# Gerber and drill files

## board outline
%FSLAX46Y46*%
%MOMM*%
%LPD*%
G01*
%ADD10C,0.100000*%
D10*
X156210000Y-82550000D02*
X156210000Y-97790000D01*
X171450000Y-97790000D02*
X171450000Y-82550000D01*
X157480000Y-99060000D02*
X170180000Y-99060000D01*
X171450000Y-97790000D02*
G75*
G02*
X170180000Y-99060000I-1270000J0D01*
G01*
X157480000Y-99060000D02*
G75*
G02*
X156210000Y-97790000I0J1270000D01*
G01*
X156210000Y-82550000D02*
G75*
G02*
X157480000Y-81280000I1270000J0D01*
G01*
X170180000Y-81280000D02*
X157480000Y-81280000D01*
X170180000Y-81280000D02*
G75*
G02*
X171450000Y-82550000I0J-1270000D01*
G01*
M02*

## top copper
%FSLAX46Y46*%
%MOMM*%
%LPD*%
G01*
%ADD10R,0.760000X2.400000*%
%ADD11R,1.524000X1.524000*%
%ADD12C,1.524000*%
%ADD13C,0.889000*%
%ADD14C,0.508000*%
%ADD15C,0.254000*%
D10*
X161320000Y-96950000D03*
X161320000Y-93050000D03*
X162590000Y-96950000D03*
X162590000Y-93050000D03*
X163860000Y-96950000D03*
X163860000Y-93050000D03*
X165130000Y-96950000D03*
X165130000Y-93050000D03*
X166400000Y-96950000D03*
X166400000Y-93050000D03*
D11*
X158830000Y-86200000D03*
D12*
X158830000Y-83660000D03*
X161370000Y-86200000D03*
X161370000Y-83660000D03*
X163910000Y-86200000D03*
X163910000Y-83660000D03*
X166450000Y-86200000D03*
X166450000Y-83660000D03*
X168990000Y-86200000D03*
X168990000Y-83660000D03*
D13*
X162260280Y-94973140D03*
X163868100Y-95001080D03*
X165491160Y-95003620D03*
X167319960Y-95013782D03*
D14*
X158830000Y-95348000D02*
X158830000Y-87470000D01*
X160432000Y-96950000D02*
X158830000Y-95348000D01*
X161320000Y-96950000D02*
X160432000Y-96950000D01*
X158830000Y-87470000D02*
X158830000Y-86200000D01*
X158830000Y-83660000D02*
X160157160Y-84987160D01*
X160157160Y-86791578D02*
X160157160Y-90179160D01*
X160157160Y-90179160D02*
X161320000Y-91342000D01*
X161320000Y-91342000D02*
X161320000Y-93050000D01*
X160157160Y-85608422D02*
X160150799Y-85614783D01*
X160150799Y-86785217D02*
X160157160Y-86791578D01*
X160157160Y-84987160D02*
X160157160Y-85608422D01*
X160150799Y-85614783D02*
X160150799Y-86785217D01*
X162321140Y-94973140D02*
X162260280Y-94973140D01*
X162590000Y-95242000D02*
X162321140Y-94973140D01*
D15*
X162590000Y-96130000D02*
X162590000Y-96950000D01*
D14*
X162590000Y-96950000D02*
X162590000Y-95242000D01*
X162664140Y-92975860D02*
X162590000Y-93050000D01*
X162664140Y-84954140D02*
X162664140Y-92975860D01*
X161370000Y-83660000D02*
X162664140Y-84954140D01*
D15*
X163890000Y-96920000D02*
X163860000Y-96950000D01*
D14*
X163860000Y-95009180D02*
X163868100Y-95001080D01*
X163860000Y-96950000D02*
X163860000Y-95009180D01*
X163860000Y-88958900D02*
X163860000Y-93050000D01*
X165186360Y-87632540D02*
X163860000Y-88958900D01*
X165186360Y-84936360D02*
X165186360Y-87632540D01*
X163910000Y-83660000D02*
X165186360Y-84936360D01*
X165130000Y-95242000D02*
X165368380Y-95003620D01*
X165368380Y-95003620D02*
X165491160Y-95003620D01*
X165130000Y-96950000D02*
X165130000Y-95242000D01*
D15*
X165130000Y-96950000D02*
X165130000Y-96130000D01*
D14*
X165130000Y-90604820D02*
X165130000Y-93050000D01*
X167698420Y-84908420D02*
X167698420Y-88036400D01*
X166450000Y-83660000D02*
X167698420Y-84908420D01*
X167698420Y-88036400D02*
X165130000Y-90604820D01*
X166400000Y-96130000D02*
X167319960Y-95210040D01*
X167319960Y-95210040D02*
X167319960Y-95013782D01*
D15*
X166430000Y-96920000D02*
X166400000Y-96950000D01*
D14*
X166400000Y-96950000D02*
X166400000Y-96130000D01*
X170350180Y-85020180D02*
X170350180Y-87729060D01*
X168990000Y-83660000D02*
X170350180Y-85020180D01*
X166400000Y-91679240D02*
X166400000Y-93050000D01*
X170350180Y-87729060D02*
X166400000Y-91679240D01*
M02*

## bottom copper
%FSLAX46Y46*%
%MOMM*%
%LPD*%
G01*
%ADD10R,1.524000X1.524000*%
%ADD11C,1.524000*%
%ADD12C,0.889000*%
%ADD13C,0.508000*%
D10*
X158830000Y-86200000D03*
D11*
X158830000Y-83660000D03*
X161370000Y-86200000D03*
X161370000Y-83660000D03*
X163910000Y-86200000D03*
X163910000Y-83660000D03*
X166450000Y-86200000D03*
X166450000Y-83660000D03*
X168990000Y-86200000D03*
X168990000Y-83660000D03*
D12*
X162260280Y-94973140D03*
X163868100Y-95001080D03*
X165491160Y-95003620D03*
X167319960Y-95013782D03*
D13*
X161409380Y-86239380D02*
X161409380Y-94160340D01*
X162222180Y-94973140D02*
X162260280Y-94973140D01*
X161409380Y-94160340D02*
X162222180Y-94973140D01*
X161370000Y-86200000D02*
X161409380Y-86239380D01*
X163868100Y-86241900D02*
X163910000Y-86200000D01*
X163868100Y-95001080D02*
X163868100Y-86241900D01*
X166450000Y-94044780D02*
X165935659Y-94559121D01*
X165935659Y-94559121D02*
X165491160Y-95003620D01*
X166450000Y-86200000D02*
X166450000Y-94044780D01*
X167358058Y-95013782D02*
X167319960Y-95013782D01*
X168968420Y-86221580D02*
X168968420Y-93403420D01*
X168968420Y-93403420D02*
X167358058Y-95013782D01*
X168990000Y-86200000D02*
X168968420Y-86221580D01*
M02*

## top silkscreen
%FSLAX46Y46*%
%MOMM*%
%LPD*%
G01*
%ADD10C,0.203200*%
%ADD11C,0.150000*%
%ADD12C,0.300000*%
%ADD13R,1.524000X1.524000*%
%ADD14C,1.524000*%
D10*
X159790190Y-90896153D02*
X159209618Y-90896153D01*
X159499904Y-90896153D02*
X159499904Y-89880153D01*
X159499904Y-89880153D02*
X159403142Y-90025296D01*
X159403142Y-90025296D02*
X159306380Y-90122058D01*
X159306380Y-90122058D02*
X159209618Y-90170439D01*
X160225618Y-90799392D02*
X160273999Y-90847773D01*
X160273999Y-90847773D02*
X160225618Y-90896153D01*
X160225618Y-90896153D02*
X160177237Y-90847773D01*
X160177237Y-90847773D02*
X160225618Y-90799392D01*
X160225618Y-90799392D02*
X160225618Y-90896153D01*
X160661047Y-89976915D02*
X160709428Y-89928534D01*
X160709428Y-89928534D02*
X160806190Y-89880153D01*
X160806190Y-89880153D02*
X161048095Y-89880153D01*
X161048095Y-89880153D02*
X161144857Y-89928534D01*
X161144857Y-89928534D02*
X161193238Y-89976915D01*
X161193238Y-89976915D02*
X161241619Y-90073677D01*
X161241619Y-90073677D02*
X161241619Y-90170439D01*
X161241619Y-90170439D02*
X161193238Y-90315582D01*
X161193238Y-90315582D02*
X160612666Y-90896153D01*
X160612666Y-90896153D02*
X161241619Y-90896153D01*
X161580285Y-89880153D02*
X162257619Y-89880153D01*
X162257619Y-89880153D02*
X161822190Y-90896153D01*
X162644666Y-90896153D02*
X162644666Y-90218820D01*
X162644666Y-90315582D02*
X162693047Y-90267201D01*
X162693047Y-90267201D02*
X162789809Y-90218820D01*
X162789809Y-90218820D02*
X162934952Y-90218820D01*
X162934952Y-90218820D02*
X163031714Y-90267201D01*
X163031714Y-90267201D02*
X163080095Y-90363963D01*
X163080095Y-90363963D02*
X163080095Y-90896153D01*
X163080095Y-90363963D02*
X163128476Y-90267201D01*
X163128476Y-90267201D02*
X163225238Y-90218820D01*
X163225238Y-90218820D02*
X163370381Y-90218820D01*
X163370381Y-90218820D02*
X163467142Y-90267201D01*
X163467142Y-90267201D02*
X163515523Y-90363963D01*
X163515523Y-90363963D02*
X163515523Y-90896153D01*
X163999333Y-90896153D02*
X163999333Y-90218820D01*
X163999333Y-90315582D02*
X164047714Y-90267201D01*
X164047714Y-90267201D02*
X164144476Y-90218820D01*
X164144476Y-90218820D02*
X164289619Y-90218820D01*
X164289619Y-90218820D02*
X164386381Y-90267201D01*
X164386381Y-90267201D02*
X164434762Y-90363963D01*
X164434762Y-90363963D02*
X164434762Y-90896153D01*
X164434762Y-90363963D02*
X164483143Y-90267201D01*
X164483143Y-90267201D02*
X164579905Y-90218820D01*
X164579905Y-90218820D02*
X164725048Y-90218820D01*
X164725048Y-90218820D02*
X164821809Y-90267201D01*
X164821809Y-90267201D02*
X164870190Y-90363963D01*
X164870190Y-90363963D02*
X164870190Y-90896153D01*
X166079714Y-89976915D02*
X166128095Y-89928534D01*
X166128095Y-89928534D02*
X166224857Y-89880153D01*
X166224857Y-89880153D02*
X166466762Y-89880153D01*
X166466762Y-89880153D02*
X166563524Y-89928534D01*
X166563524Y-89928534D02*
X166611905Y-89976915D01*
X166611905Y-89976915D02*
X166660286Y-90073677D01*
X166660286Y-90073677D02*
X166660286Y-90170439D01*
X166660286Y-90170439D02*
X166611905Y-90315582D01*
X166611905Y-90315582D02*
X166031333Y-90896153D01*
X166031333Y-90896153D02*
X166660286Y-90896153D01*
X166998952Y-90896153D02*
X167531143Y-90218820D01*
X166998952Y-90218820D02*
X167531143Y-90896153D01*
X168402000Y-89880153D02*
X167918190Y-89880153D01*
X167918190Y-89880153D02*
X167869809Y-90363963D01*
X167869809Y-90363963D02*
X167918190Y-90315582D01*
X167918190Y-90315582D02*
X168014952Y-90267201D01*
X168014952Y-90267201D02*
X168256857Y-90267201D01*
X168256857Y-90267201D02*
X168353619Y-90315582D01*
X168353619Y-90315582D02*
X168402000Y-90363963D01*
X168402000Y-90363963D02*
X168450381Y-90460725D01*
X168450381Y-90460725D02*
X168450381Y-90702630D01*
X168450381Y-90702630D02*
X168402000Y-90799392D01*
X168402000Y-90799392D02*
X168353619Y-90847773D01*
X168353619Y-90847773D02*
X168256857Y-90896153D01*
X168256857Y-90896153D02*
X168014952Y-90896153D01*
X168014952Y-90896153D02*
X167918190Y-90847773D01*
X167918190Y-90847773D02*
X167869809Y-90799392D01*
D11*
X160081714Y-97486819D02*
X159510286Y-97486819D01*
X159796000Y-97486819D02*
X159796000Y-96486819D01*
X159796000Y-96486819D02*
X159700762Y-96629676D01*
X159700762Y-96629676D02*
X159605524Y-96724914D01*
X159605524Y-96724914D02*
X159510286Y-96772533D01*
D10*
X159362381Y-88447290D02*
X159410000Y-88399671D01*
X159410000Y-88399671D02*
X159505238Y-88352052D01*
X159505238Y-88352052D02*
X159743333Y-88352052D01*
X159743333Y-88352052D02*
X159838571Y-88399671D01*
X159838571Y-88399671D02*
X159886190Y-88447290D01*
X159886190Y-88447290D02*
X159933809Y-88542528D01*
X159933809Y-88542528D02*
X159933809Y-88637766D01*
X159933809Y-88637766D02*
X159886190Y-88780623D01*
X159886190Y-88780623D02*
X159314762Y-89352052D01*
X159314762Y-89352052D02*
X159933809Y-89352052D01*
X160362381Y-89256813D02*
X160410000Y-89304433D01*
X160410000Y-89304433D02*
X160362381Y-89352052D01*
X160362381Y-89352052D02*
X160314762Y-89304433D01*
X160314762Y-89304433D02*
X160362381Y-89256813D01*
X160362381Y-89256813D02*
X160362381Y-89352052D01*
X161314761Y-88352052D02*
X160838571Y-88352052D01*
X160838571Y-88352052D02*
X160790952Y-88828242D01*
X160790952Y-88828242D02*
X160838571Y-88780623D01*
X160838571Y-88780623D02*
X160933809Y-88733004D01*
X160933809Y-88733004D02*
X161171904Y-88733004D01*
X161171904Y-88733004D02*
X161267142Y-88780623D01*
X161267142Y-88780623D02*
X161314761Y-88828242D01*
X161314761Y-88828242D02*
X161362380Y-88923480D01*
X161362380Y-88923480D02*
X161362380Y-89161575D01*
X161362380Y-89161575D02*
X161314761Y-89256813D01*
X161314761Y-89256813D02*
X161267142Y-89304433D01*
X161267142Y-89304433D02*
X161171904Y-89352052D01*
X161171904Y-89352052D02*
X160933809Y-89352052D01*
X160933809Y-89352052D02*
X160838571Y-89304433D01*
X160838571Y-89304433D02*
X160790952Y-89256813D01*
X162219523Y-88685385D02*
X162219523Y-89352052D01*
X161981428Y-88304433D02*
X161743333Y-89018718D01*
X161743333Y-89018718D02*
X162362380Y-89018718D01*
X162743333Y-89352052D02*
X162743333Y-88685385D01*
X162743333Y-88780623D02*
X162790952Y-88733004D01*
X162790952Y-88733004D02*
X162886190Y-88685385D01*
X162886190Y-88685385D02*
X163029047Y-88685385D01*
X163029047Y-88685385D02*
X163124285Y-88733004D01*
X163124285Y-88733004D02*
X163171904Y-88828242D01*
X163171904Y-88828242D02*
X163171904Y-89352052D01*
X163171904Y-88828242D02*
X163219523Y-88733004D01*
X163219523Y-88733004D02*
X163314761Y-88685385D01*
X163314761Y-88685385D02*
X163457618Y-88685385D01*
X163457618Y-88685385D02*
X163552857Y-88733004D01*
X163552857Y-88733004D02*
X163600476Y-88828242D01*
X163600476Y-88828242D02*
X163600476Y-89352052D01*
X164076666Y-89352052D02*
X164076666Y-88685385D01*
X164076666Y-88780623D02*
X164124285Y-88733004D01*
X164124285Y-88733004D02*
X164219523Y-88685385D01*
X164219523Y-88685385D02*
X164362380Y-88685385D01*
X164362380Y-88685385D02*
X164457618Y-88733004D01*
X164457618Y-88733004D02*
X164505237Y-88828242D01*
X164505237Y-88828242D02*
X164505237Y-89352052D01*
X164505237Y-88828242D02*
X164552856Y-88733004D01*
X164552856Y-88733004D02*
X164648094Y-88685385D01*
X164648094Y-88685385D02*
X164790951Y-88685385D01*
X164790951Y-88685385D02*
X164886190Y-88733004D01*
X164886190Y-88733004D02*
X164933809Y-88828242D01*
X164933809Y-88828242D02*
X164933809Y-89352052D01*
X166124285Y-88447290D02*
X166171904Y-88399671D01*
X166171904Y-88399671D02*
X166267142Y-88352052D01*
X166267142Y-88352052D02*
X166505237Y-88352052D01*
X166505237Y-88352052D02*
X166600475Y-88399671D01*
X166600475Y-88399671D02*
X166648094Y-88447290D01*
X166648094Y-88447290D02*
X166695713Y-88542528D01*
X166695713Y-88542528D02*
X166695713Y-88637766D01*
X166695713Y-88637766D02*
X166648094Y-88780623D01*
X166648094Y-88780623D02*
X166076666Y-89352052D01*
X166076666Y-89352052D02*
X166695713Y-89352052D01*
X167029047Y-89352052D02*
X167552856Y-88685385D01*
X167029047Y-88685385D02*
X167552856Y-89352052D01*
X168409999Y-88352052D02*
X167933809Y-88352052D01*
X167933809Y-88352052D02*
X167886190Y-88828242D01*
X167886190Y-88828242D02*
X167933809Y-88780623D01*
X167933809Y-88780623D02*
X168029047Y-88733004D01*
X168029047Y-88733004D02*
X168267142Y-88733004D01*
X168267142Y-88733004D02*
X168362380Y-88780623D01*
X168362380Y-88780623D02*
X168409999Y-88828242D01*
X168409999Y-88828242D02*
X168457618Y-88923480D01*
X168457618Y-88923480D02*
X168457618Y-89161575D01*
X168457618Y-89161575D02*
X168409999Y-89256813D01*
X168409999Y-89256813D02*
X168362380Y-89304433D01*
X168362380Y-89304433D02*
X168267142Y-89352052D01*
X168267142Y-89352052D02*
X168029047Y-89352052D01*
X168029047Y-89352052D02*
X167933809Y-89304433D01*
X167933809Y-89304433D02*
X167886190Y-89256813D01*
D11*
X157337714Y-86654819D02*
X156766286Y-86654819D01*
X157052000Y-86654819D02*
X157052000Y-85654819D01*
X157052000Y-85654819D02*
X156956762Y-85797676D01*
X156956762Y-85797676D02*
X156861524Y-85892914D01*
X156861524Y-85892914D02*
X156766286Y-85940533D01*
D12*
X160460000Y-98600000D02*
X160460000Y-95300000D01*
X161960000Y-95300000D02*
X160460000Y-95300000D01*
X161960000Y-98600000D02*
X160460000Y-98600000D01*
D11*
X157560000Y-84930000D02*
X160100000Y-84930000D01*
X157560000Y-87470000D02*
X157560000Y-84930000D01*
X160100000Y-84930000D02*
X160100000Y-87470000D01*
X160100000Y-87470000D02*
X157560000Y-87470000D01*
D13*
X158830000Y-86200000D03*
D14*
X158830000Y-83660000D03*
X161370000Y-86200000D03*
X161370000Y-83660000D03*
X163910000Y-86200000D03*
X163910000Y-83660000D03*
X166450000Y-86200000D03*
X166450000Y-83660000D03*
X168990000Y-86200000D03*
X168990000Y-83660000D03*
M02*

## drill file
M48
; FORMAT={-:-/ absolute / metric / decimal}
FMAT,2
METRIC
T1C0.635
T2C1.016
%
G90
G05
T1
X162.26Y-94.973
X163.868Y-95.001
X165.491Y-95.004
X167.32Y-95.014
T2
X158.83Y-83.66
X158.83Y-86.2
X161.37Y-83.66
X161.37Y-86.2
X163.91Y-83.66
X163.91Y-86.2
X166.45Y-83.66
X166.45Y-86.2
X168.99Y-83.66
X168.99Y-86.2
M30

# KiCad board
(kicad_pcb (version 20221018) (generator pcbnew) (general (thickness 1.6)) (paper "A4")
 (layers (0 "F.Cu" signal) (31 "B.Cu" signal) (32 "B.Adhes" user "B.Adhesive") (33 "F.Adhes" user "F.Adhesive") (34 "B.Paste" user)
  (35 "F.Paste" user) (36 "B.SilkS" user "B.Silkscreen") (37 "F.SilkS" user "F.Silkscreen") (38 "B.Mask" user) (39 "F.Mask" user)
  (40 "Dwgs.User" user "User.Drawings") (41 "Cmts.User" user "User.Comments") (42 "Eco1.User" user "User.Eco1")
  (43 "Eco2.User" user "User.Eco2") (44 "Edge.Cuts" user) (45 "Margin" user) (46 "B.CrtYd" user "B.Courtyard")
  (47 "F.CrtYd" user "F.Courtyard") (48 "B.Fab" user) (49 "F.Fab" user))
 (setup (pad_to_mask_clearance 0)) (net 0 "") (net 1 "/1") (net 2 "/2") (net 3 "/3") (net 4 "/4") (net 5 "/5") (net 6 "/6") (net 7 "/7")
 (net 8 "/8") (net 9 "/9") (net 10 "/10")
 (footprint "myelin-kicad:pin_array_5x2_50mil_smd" (layer "F.Cu") (at 163.86 95)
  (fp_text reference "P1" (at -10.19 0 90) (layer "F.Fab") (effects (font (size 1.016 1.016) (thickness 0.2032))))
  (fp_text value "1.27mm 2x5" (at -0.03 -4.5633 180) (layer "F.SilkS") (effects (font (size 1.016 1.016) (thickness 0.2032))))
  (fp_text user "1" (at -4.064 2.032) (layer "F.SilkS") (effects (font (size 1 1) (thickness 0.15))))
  (fp_line (start -3.4 3.6) (end -3.4 0.3) (stroke (width 0.3) (type solid)) (layer "F.SilkS"))
  (fp_line (start -1.9 0.3) (end -3.4 0.3) (stroke (width 0.3) (type solid)) (layer "F.SilkS"))
  (fp_line (start -1.9 3.6) (end -3.4 3.6) (stroke (width 0.3) (type solid)) (layer "F.SilkS"))
  (pad "1" smd rect (at -2.54 1.95) (size 0.76 2.4) (layers "F.Cu" "F.Paste" "F.Mask") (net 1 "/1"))
  (pad "2" smd rect (at -2.54 -1.95) (size 0.76 2.4) (layers "F.Cu" "F.Paste" "F.Mask") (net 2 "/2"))
  (pad "3" smd rect (at -1.27 1.95) (size 0.76 2.4) (layers "F.Cu" "F.Paste" "F.Mask") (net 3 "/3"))
  (pad "4" smd rect (at -1.27 -1.95) (size 0.76 2.4) (layers "F.Cu" "F.Paste" "F.Mask") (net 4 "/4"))
  (pad "5" smd rect (at 0 1.95) (size 0.76 2.4) (layers "F.Cu" "F.Paste" "F.Mask") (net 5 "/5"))
  (pad "6" smd rect (at 0 -1.95) (size 0.76 2.4) (layers "F.Cu" "F.Paste" "F.Mask") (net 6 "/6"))
  (pad "7" smd rect (at 1.27 1.95) (size 0.76 2.4) (layers "F.Cu" "F.Paste" "F.Mask") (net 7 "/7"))
  (pad "8" smd rect (at 1.27 -1.95) (size 0.76 2.4) (layers "F.Cu" "F.Paste" "F.Mask") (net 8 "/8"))
  (pad "9" smd rect (at 2.54 1.95) (size 0.76 2.4) (layers "F.Cu" "F.Paste" "F.Mask") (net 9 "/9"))
  (pad "10" smd rect (at 2.54 -1.95) (size 0.76 2.4) (layers "F.Cu" "F.Paste" "F.Mask") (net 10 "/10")))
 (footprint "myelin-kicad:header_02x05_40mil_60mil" (layer "F.Cu") (at 163.91 84.93)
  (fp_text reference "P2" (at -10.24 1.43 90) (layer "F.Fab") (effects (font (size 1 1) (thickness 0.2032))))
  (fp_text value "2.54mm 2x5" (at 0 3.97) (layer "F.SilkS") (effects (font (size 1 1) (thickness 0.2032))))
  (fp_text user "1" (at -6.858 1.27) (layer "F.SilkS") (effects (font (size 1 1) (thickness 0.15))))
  (fp_line (start -6.35 0) (end -3.81 0) (stroke (width 0.15) (type solid)) (layer "F.SilkS"))
  (fp_line (start -6.35 2.54) (end -6.35 0) (stroke (width 0.15) (type solid)) (layer "F.SilkS"))
  (fp_line (start -3.81 0) (end -3.81 2.54) (stroke (width 0.15) (type solid)) (layer "F.SilkS"))
  (fp_line (start -3.81 2.54) (end -6.35 2.54) (stroke (width 0.15) (type solid)) (layer "F.SilkS"))
  (pad "1" thru_hole rect (at -5.08 1.27) (size 1.524 1.524) (drill 1.016) (layers "*.Cu" "*.Mask" "F.SilkS") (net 1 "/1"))
  (pad "2" thru_hole circle (at -5.08 -1.27) (size 1.524 1.524) (drill 1.016) (layers "*.Cu" "*.Mask" "F.SilkS") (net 2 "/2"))
  (pad "3" thru_hole circle (at -2.54 1.27) (size 1.524 1.524) (drill 1.016) (layers "*.Cu" "*.Mask" "F.SilkS") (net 3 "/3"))
  (pad "4" thru_hole circle (at -2.54 -1.27) (size 1.524 1.524) (drill 1.016) (layers "*.Cu" "*.Mask" "F.SilkS") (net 4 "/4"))
  (pad "5" thru_hole circle (at 0 1.27) (size 1.524 1.524) (drill 1.016) (layers "*.Cu" "*.Mask" "F.SilkS") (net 5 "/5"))
  (pad "6" thru_hole circle (at 0 -1.27) (size 1.524 1.524) (drill 1.016) (layers "*.Cu" "*.Mask" "F.SilkS") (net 6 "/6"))
  (pad "7" thru_hole circle (at 2.54 1.27) (size 1.524 1.524) (drill 1.016) (layers "*.Cu" "*.Mask" "F.SilkS") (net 7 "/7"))
  (pad "8" thru_hole circle (at 2.54 -1.27) (size 1.524 1.524) (drill 1.016) (layers "*.Cu" "*.Mask" "F.SilkS") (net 8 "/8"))
  (pad "9" thru_hole circle (at 5.08 1.27) (size 1.524 1.524) (drill 1.016) (layers "*.Cu" "*.Mask" "F.SilkS") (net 9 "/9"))
  (pad "10" thru_hole circle (at 5.08 -1.27) (size 1.524 1.524) (drill 1.016) (layers "*.Cu" "*.Mask" "F.SilkS") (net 10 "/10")))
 (gr_line (start 156.21 82.55) (end 156.21 97.79) (stroke (width 0.1) (type solid)) (layer "Edge.Cuts"))
 (gr_line (start 171.45 97.79) (end 171.45 82.55) (stroke (width 0.1) (type solid)) (layer "Edge.Cuts"))
 (gr_line (start 157.48 99.06) (end 170.18 99.06) (stroke (width 0.1) (type solid)) (layer "Edge.Cuts"))
 (gr_arc (start 171.45 97.79) (mid 171.078026 98.688026) (end 170.18 99.06) (stroke (width 0.1) (type solid)) (layer "Edge.Cuts"))
 (gr_arc (start 157.48 99.06) (mid 156.581974 98.688026) (end 156.21 97.79) (stroke (width 0.1) (type solid)) (layer "Edge.Cuts"))
 (gr_arc (start 156.21 82.55) (mid 156.581974 81.651974) (end 157.48 81.28) (stroke (width 0.1) (type solid)) (layer "Edge.Cuts"))
 (gr_line (start 170.18 81.28) (end 157.48 81.28) (stroke (width 0.1) (type solid)) (layer "Edge.Cuts"))
 (gr_arc (start 170.18 81.28) (mid 171.078026 81.651974) (end 171.45 82.55) (stroke (width 0.1) (type solid)) (layer "Edge.Cuts"))
 (segment (start 158.83 95.348) (end 158.83 87.47) (width 0.508) (layer "F.Cu") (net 1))
 (segment (start 160.432 96.95) (end 158.83 95.348) (width 0.508) (layer "F.Cu") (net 1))
 (segment (start 161.32 96.95) (end 160.432 96.95) (width 0.508) (layer "F.Cu") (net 1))
 (segment (start 158.83 87.47) (end 158.83 86.2) (width 0.508) (layer "F.Cu") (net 1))
 (segment (start 158.83 83.66) (end 160.15716 84.98716) (width 0.508) (layer "F.Cu") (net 2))
 (segment (start 160.15716 86.791578) (end 160.15716 90.17916) (width 0.508) (layer "F.Cu") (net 2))
 (segment (start 160.15716 90.17916) (end 161.32 91.342) (width 0.508) (layer "F.Cu") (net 2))
 (segment (start 161.32 91.342) (end 161.32 93.05) (width 0.508) (layer "F.Cu") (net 2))
 (segment (start 160.15716 85.608422) (end 160.150799 85.614783) (width 0.508) (layer "F.Cu") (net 2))
 (segment (start 160.150799 86.785217) (end 160.15716 86.791578) (width 0.508) (layer "F.Cu") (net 2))
 (segment (start 160.15716 84.98716) (end 160.15716 85.608422) (width 0.508) (layer "F.Cu") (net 2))
 (segment (start 160.150799 85.614783) (end 160.150799 86.785217) (width 0.508) (layer "F.Cu") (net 2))
 (segment (start 162.32114 94.97314) (end 162.26028 94.97314) (width 0.508) (layer "F.Cu") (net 3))
 (segment (start 162.59 95.242) (end 162.32114 94.97314) (width 0.508) (layer "F.Cu") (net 3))
 (segment (start 162.59 96.13) (end 162.59 96.95) (width 0.254) (layer "F.Cu") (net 3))
 (segment (start 162.59 96.95) (end 162.59 95.242) (width 0.508) (layer "F.Cu") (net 3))
 (via (at 162.26028 94.97314) (size 0.889) (drill 0.635) (layers "F.Cu" "B.Cu") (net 3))
 (segment (start 161.40938 86.23938) (end 161.40938 94.16034) (width 0.508) (layer "B.Cu") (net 3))
 (segment (start 162.22218 94.97314) (end 162.26028 94.97314) (width 0.508) (layer "B.Cu") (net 3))
 (segment (start 161.40938 94.16034) (end 162.22218 94.97314) (width 0.508) (layer "B.Cu") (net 3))
 (segment (start 161.37 86.2) (end 161.40938 86.23938) (width 0.508) (layer "B.Cu") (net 3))
 (segment (start 162.66414 92.97586) (end 162.59 93.05) (width 0.508) (layer "F.Cu") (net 4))
 (segment (start 162.66414 84.95414) (end 162.66414 92.97586) (width 0.508) (layer "F.Cu") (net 4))
 (segment (start 161.37 83.66) (end 162.66414 84.95414) (width 0.508) (layer "F.Cu") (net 4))
 (segment (start 163.89 96.92) (end 163.86 96.95) (width 0.254) (layer "F.Cu") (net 5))
 (segment (start 163.86 95.00918) (end 163.8681 95.00108) (width 0.508) (layer "F.Cu") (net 5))
 (segment (start 163.86 96.95) (end 163.86 95.00918) (width 0.508) (layer "F.Cu") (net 5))
 (via (at 163.8681 95.00108) (size 0.889) (drill 0.635) (layers "F.Cu" "B.Cu") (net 5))
 (segment (start 163.8681 86.2419) (end 163.91 86.2) (width 0.508) (layer "B.Cu") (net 5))
 (segment (start 163.8681 95.00108) (end 163.8681 86.2419) (width 0.508) (layer "B.Cu") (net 5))
 (segment (start 163.86 88.9589) (end 163.86 93.05) (width 0.508) (layer "F.Cu") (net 6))
 (segment (start 165.18636 87.63254) (end 163.86 88.9589) (width 0.508) (layer "F.Cu") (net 6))
 (segment (start 165.18636 84.93636) (end 165.18636 87.63254) (width 0.508) (layer "F.Cu") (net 6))
 (segment (start 163.91 83.66) (end 165.18636 84.93636) (width 0.508) (layer "F.Cu") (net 6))
 (segment (start 165.13 95.242) (end 165.36838 95.00362) (width 0.508) (layer "F.Cu") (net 7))
 (segment (start 165.36838 95.00362) (end 165.49116 95.00362) (width 0.508) (layer "F.Cu") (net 7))
 (segment (start 165.13 96.95) (end 165.13 95.242) (width 0.508) (layer "F.Cu") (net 7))
 (segment (start 165.13 96.95) (end 165.13 96.13) (width 0.254) (layer "F.Cu") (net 7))
 (via (at 165.49116 95.00362) (size 0.889) (drill 0.635) (layers "F.Cu" "B.Cu") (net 7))
 (segment (start 166.45 94.04478) (end 165.935659 94.559121) (width 0.508) (layer "B.Cu") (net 7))
 (segment (start 165.935659 94.559121) (end 165.49116 95.00362) (width 0.508) (layer "B.Cu") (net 7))
 (segment (start 166.45 86.2) (end 166.45 94.04478) (width 0.508) (layer "B.Cu") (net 7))
 (segment (start 165.13 90.60482) (end 165.13 93.05) (width 0.508) (layer "F.Cu") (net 8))
 (segment (start 167.69842 84.90842) (end 167.69842 88.0364) (width 0.508) (layer "F.Cu") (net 8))
 (segment (start 166.45 83.66) (end 167.69842 84.90842) (width 0.508) (layer "F.Cu") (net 8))
 (segment (start 167.69842 88.0364) (end 165.13 90.60482) (width 0.508) (layer "F.Cu") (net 8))
 (segment (start 166.4 96.13) (end 167.31996 95.21004) (width 0.508) (layer "F.Cu") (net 9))
 (segment (start 167.31996 95.21004) (end 167.31996 95.013782) (width 0.508) (layer "F.Cu") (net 9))
 (segment (start 166.43 96.92) (end 166.4 96.95) (width 0.254) (layer "F.Cu") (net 9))
 (segment (start 166.4 96.95) (end 166.4 96.13) (width 0.508) (layer "F.Cu") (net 9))
 (via (at 167.31996 95.013782) (size 0.889) (drill 0.635) (layers "F.Cu" "B.Cu") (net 9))
 (segment (start 167.358058 95.013782) (end 167.31996 95.013782) (width 0.508) (layer "B.Cu") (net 9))
 (segment (start 168.96842 86.22158) (end 168.96842 93.40342) (width 0.508) (layer "B.Cu") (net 9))
 (segment (start 168.96842 93.40342) (end 167.358058 95.013782) (width 0.508) (layer "B.Cu") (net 9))
 (segment (start 168.99 86.2) (end 168.96842 86.22158) (width 0.508) (layer "B.Cu") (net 9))
 (segment (start 170.35018 85.02018) (end 170.35018 87.72906) (width 0.508) (layer "F.Cu") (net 10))
 (segment (start 168.99 83.66) (end 170.35018 85.02018) (width 0.508) (layer "F.Cu") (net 10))
 (segment (start 166.4 91.67924) (end 166.4 93.05) (width 0.508) (layer "F.Cu") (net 10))
 (segment (start 170.35018 87.72906) (end 166.4 91.67924) (width 0.508) (layer "F.Cu") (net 10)))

